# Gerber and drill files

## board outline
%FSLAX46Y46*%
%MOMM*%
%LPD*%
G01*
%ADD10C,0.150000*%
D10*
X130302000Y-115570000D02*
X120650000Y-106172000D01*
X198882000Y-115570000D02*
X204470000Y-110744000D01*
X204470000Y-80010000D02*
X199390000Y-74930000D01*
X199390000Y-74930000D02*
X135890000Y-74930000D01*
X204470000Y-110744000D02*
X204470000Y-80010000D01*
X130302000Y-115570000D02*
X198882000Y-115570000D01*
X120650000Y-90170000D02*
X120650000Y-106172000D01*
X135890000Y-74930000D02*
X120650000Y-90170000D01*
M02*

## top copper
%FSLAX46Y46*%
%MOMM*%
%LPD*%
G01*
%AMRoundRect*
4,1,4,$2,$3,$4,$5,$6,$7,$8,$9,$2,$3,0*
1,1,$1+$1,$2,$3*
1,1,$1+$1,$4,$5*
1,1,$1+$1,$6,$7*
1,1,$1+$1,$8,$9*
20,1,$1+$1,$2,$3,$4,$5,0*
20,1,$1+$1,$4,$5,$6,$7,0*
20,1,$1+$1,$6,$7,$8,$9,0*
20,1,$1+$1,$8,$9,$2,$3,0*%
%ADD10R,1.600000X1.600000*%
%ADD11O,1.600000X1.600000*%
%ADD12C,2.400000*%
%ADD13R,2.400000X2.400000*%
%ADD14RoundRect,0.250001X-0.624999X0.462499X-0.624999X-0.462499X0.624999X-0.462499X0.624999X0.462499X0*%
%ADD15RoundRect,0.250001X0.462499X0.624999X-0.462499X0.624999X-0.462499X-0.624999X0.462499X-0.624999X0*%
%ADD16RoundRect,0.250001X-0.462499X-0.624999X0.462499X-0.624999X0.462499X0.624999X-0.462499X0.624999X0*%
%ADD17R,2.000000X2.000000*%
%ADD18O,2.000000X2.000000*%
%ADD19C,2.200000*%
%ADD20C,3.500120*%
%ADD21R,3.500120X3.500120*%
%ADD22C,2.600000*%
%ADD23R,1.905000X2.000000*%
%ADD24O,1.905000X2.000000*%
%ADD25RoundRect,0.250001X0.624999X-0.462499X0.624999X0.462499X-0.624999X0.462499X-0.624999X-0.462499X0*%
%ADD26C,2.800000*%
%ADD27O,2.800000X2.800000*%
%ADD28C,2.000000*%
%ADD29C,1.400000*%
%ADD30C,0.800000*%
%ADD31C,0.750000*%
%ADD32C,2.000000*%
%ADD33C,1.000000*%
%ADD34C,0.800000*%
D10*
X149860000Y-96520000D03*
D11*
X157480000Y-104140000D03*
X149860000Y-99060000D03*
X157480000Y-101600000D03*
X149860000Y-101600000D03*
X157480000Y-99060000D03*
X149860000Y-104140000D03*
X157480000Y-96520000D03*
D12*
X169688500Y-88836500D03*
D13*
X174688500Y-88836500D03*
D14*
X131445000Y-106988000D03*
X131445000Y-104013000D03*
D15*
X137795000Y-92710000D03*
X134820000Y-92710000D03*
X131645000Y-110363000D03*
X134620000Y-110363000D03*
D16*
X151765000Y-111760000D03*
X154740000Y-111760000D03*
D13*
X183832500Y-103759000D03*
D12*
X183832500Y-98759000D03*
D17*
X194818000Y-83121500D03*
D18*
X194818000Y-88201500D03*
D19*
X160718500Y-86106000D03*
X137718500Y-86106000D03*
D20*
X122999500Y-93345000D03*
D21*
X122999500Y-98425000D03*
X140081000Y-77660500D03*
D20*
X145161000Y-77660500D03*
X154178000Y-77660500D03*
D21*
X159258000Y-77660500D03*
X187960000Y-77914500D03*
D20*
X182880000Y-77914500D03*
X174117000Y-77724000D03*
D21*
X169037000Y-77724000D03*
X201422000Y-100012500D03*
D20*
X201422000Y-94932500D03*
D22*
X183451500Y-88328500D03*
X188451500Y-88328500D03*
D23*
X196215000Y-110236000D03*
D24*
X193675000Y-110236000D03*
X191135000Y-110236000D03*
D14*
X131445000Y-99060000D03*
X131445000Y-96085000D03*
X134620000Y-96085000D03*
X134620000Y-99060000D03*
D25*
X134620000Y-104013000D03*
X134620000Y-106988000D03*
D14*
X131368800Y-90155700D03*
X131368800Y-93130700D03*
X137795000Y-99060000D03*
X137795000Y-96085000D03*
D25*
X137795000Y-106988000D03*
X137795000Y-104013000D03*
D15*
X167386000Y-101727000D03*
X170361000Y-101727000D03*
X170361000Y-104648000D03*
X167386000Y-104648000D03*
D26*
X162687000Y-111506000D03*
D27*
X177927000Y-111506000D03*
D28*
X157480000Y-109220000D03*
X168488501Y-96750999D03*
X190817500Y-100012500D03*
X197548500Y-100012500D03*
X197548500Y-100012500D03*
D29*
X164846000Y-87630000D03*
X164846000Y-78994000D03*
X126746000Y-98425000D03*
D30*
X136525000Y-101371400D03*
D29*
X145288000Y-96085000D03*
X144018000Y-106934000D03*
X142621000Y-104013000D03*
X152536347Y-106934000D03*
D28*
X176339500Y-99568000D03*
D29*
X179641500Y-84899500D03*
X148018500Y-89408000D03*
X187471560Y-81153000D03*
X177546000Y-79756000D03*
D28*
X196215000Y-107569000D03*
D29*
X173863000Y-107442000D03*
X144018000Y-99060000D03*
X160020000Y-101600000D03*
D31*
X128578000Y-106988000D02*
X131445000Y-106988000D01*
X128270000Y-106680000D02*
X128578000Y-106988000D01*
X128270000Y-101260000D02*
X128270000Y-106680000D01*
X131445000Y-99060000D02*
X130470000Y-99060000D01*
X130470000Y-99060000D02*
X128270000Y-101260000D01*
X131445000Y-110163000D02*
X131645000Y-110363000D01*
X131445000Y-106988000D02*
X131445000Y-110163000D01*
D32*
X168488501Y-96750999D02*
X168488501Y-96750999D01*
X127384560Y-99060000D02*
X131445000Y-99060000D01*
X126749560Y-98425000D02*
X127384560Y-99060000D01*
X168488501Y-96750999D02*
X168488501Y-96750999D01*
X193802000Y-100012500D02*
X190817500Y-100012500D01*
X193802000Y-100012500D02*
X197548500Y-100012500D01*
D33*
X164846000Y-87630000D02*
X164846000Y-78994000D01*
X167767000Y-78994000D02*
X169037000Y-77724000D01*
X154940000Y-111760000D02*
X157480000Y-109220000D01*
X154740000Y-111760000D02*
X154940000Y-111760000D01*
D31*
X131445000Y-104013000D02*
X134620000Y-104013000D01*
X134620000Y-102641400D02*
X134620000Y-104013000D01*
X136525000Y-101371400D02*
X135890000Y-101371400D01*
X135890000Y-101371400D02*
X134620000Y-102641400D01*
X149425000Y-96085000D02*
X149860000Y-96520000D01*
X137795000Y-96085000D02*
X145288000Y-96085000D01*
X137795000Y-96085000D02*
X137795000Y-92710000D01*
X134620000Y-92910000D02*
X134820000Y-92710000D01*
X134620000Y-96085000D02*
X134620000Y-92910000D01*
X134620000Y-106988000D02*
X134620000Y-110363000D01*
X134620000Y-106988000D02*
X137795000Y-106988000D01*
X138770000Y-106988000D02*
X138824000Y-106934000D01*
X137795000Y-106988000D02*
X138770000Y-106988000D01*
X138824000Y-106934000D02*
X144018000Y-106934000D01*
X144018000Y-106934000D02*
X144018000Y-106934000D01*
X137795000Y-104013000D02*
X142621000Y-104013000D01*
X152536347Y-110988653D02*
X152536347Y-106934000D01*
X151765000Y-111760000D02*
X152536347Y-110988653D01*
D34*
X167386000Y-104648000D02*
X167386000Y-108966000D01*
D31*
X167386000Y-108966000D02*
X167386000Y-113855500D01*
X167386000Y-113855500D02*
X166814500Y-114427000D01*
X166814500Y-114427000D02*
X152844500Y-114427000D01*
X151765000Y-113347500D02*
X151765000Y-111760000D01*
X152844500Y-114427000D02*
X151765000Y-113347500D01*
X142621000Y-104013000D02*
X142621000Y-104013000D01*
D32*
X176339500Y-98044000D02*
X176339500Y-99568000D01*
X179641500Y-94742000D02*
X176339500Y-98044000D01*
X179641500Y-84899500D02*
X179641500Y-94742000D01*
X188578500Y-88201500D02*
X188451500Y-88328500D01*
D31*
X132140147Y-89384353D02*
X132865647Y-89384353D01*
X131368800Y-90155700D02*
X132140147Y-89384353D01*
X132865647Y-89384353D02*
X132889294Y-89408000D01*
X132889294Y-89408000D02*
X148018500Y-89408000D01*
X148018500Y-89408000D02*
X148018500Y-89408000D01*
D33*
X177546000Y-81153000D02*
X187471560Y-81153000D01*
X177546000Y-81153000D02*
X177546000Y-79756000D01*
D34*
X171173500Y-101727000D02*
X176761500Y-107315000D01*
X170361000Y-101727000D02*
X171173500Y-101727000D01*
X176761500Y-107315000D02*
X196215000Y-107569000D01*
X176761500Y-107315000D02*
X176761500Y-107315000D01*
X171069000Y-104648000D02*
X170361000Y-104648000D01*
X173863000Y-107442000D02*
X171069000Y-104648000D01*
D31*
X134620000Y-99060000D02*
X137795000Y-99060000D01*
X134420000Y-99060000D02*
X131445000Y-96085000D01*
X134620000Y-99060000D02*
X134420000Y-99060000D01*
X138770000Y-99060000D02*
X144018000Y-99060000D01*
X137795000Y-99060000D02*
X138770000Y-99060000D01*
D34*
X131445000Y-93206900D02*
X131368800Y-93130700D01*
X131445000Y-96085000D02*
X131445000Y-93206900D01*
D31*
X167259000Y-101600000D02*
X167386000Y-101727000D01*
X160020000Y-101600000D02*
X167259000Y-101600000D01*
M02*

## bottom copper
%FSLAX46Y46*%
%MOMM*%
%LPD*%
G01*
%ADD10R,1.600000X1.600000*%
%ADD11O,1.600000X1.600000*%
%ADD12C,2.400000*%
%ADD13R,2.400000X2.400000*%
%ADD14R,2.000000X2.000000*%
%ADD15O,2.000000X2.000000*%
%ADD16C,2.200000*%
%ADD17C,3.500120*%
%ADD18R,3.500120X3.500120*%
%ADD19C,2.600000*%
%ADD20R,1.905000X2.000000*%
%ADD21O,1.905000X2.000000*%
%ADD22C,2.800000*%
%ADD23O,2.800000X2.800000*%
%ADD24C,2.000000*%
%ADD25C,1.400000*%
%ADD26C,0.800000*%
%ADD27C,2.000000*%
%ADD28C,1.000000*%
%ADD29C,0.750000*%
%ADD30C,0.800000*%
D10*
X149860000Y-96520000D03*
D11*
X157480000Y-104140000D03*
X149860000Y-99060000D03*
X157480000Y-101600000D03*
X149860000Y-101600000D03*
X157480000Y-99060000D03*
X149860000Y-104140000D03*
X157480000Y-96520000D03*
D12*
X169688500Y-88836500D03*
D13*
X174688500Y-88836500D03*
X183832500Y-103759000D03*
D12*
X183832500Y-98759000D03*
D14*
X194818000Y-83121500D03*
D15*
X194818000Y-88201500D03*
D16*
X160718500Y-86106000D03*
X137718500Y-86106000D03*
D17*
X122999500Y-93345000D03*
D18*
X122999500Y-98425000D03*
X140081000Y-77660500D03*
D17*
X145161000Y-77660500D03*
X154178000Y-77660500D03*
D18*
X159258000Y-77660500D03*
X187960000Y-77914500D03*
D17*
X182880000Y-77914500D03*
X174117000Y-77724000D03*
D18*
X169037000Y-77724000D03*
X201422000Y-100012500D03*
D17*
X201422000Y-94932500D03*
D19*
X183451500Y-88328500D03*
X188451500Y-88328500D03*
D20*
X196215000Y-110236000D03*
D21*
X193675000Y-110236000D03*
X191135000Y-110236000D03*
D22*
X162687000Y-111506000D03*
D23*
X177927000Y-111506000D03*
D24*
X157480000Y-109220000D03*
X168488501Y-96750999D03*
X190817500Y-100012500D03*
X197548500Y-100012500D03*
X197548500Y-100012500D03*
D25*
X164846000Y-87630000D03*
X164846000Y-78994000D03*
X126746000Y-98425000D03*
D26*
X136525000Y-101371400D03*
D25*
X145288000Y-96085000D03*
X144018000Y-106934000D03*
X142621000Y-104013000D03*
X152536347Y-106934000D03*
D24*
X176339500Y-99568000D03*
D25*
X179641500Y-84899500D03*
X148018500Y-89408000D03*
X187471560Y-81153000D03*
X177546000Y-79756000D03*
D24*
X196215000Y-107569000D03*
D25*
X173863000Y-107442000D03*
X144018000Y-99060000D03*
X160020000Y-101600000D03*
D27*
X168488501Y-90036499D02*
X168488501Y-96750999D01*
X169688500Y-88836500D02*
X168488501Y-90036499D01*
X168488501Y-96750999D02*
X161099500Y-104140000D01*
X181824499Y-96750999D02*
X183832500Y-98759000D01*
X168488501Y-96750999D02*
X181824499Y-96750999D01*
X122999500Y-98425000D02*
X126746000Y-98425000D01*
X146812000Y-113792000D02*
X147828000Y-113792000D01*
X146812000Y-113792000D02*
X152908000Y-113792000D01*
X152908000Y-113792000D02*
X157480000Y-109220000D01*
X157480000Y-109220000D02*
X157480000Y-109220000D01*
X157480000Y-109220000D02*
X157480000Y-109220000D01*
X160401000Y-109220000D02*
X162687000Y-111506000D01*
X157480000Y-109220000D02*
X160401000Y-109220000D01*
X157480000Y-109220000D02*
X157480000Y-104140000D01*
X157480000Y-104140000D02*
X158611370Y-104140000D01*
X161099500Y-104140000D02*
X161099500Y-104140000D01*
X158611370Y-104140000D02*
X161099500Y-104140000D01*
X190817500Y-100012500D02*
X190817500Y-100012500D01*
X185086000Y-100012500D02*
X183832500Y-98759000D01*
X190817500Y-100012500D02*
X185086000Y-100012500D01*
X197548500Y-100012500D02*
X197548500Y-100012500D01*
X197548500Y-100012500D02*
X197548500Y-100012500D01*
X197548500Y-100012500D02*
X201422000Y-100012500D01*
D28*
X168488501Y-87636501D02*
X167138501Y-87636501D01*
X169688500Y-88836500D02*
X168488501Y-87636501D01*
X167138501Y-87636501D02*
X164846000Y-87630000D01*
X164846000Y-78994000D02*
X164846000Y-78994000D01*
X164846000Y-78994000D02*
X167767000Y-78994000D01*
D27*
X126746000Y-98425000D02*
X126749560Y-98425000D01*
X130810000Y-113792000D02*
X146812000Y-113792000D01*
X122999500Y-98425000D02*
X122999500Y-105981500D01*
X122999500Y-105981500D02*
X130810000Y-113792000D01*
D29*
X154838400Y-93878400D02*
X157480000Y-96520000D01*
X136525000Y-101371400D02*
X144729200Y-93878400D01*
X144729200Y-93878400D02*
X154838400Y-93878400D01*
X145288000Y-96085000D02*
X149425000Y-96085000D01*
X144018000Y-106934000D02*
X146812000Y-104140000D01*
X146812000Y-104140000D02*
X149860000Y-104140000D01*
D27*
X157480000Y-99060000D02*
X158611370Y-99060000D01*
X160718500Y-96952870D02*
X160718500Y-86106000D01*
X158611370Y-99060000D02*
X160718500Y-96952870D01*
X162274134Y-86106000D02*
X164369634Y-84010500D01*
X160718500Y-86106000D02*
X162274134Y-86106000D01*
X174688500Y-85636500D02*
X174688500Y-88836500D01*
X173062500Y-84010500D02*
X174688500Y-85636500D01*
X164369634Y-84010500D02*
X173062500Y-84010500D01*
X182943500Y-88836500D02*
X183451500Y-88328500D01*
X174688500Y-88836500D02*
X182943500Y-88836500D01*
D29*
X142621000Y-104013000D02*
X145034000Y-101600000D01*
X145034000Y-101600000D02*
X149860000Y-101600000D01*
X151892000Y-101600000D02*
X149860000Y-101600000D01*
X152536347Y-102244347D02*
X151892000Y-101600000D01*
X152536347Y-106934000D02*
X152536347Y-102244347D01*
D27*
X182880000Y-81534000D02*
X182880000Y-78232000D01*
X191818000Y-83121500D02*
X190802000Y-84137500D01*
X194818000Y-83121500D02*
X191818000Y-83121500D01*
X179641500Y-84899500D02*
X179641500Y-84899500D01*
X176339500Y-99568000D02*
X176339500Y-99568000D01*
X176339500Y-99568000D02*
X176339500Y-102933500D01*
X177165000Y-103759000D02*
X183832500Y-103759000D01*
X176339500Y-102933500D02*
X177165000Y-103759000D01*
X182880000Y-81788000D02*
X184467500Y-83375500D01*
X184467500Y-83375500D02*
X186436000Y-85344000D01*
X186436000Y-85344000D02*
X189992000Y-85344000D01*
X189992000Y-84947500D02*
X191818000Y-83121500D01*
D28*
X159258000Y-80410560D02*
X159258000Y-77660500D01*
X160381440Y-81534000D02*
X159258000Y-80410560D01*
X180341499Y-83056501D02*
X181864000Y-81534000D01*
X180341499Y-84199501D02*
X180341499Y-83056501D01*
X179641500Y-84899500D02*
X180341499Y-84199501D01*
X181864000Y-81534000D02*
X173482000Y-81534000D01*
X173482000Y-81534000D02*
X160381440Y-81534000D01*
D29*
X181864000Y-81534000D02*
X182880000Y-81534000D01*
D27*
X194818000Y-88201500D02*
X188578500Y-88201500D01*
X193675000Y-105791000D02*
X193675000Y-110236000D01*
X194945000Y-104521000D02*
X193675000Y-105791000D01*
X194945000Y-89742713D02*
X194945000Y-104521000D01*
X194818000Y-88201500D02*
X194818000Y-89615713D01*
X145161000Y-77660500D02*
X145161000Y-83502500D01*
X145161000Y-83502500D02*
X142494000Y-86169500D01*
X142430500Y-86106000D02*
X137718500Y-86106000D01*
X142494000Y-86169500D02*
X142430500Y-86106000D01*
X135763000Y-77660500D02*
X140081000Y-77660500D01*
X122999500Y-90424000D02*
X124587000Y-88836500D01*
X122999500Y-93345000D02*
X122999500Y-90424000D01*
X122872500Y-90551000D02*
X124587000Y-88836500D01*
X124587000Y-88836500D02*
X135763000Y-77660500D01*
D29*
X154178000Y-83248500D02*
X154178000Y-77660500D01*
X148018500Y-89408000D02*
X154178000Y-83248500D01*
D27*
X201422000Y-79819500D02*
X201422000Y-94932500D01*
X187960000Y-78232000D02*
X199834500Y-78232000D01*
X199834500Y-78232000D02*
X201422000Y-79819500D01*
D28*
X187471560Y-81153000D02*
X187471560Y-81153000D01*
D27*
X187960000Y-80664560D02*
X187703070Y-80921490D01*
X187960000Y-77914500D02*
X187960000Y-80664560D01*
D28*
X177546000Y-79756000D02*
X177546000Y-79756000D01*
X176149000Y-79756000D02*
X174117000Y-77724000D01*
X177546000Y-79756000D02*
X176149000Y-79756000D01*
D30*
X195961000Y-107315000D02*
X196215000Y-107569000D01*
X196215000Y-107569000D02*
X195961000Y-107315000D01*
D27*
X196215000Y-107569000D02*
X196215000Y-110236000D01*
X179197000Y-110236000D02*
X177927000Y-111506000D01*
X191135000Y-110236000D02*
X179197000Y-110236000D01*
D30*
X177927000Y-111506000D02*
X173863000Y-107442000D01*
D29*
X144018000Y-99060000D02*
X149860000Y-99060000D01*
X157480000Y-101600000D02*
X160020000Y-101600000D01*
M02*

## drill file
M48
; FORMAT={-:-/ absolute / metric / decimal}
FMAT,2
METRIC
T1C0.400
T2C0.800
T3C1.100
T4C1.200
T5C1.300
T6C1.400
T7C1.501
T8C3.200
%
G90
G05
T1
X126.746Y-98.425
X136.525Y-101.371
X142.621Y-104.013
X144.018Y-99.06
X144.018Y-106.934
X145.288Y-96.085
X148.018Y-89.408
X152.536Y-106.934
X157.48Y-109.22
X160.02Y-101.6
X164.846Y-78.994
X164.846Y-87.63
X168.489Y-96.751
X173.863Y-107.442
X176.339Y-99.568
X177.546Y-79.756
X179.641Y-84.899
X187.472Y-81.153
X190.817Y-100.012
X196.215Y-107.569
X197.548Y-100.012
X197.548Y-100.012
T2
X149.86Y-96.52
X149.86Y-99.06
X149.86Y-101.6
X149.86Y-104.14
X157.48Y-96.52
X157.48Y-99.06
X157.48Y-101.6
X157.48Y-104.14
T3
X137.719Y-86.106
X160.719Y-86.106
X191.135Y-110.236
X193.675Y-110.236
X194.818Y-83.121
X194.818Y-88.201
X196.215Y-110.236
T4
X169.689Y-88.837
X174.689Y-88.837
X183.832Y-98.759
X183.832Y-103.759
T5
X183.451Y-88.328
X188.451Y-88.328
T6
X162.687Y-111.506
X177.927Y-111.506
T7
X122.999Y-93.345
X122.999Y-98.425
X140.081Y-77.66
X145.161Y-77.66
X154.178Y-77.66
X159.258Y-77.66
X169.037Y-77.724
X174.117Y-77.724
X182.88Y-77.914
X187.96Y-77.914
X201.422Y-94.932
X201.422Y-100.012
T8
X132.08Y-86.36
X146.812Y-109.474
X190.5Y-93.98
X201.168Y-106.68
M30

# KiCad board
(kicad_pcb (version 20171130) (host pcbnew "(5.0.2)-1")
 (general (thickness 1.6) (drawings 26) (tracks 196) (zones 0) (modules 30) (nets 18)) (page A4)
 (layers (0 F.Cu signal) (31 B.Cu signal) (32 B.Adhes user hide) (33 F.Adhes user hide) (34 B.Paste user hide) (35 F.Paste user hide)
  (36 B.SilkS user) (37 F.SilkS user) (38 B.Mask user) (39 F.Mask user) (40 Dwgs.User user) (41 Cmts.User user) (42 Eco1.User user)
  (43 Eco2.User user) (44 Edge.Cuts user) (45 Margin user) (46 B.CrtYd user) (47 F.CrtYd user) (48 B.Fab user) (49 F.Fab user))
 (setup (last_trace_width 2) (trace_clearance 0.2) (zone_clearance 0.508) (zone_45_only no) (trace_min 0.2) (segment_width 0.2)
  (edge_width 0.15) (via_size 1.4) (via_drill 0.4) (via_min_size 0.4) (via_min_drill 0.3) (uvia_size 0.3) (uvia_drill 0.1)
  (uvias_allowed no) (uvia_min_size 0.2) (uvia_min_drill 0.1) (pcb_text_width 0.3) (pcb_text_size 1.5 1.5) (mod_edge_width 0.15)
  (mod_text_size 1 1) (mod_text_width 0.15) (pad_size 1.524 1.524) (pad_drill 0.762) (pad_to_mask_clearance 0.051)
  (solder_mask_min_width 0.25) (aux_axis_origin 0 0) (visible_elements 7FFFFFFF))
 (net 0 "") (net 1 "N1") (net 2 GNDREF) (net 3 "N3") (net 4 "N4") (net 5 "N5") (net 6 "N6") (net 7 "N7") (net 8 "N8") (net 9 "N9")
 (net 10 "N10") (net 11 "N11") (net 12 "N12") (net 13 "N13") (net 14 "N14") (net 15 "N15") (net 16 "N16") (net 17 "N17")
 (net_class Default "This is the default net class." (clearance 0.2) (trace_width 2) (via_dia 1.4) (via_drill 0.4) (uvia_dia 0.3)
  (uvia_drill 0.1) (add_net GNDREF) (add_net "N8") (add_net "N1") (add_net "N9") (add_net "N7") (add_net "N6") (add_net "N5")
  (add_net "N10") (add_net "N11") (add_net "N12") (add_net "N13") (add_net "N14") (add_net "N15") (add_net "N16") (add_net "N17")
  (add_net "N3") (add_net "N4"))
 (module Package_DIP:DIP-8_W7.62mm (layer F.Cu) (at 149.86 96.52)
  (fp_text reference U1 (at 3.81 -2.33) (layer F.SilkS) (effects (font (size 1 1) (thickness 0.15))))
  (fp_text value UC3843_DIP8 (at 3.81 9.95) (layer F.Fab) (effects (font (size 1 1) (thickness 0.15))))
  (pad 1 thru_hole rect (at 0 0) (size 1.6 1.6) (drill 0.8) (layers *.Cu *.Mask) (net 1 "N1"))
  (pad 5 thru_hole oval (at 7.62 7.62) (size 1.6 1.6) (drill 0.8) (layers *.Cu *.Mask) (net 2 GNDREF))
  (pad 2 thru_hole oval (at 0 2.54) (size 1.6 1.6) (drill 0.8) (layers *.Cu *.Mask) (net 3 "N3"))
  (pad 6 thru_hole oval (at 7.62 5.08) (size 1.6 1.6) (drill 0.8) (layers *.Cu *.Mask) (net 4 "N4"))
  (pad 3 thru_hole oval (at 0 5.08) (size 1.6 1.6) (drill 0.8) (layers *.Cu *.Mask) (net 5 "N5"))
  (pad 7 thru_hole oval (at 7.62 2.54) (size 1.6 1.6) (drill 0.8) (layers *.Cu *.Mask) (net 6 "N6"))
  (pad 4 thru_hole oval (at 0 7.62) (size 1.6 1.6) (drill 0.8) (layers *.Cu *.Mask) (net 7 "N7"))
  (pad 8 thru_hole oval (at 7.62 0) (size 1.6 1.6) (drill 0.8) (layers *.Cu *.Mask) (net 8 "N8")))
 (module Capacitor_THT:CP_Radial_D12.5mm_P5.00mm (layer F.Cu) (at 174.6885 88.8365 180)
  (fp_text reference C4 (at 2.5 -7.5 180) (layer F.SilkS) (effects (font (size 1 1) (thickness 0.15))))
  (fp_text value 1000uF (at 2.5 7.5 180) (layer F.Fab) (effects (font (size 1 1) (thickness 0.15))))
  (pad 2 thru_hole circle (at 5 0 180) (size 2.4 2.4) (drill 1.2) (layers *.Cu *.Mask) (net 2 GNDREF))
  (pad 1 thru_hole rect (at 0 0 180) (size 2.4 2.4) (drill 1.2) (layers *.Cu *.Mask) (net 6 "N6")))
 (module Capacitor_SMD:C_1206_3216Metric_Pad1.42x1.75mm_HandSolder (layer F.Cu) (at 131.445 105.5005 270)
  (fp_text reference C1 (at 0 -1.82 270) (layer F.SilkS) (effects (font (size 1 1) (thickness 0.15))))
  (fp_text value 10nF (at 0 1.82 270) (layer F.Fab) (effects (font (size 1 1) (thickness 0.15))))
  (pad 2 smd roundrect (at 1.4875 0 270) (size 1.425 1.75) (layers F.Cu F.Paste F.Mask) (roundrect_rratio 0.175439) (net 2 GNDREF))
  (pad 1 smd roundrect (at -1.4875 0 270) (size 1.425 1.75) (layers F.Cu F.Paste F.Mask) (roundrect_rratio 0.175439) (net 8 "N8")))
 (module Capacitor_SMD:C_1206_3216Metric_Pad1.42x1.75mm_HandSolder (layer F.Cu) (at 136.3075 92.71 180)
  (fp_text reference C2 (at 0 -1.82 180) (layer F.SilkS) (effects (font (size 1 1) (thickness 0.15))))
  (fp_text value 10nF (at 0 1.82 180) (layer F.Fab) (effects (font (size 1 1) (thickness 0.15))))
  (pad 1 smd roundrect (at -1.4875 0 180) (size 1.425 1.75) (layers F.Cu F.Paste F.Mask) (roundrect_rratio 0.175439) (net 1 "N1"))
  (pad 2 smd roundrect (at 1.4875 0 180) (size 1.425 1.75) (layers F.Cu F.Paste F.Mask) (roundrect_rratio 0.175439) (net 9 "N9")))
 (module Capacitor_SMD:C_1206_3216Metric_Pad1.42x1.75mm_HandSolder (layer F.Cu) (at 133.1325 110.363 180)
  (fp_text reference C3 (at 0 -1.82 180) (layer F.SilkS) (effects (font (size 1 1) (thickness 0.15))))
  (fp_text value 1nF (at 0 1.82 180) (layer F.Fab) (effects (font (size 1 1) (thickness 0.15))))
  (pad 2 smd roundrect (at 1.4875 0 180) (size 1.425 1.75) (layers F.Cu F.Paste F.Mask) (roundrect_rratio 0.175439) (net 2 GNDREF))
  (pad 1 smd roundrect (at -1.4875 0 180) (size 1.425 1.75) (layers F.Cu F.Paste F.Mask) (roundrect_rratio 0.175439) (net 7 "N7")))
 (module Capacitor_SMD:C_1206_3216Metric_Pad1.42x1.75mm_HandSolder (layer F.Cu) (at 153.2525 111.76)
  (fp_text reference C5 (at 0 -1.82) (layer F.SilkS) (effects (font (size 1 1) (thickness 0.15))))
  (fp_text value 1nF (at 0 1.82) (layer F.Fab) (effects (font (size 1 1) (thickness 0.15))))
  (pad 1 smd roundrect (at -1.4875 0) (size 1.425 1.75) (layers F.Cu F.Paste F.Mask) (roundrect_rratio 0.175439) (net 5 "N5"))
  (pad 2 smd roundrect (at 1.4875 0) (size 1.425 1.75) (layers F.Cu F.Paste F.Mask) (roundrect_rratio 0.175439) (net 2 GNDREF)))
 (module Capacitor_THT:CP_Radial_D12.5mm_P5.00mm (layer F.Cu) (at 183.8325 103.759 90)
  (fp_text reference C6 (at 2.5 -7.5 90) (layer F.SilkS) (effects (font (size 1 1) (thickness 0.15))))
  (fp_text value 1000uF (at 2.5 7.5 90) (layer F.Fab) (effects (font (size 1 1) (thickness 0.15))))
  (pad 1 thru_hole rect (at 0 0 90) (size 2.4 2.4) (drill 1.2) (layers *.Cu *.Mask) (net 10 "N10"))
  (pad 2 thru_hole circle (at 5 0 90) (size 2.4 2.4) (drill 1.2) (layers *.Cu *.Mask) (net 2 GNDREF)))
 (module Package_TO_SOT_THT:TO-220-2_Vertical (layer F.Cu) (at 194.818 83.1215 270)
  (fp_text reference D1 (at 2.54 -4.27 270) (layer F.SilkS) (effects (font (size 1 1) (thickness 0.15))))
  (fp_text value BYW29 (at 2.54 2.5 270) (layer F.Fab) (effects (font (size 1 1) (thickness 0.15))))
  (pad 1 thru_hole rect (at 0 0 270) (size 2 2) (drill 1.1) (layers *.Cu *.Mask) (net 10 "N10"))
  (pad 2 thru_hole oval (at 5.08 0 270) (size 2 2) (drill 1.1) (layers *.Cu *.Mask) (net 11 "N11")))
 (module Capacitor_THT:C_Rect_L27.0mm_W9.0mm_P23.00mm (layer F.Cu) (at 160.7185 86.106 180)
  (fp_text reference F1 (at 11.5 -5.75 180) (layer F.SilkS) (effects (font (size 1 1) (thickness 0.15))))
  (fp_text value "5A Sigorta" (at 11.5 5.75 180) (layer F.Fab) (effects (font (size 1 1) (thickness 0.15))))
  (pad 1 thru_hole circle (at 0 0 180) (size 2.2 2.2) (drill 1.1) (layers *.Cu *.Mask) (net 6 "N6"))
  (pad 2 thru_hole circle (at 23 0 180) (size 2.2 2.2) (drill 1.1) (layers *.Cu *.Mask) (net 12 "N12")))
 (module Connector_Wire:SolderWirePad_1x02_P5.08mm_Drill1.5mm (layer F.Cu) (at 122.9995 98.425 90)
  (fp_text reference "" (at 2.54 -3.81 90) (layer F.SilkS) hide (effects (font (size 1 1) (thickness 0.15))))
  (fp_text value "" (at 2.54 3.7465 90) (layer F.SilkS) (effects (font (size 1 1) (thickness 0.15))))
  (pad 2 thru_hole circle (at 5.08 0 90) (size 3.50012 3.50012) (drill 1.50114) (layers *.Cu *.Mask) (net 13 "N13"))
  (pad 1 thru_hole rect (at 0 0 90) (size 3.50012 3.50012) (drill 1.50114) (layers *.Cu *.Mask) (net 2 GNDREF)))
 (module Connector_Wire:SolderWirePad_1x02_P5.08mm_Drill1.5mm (layer F.Cu) (at 140.081 77.6605)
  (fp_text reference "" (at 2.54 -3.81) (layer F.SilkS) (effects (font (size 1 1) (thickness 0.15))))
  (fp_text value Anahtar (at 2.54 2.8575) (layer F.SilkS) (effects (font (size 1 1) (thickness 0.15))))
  (pad 1 thru_hole rect (at 0 0) (size 3.50012 3.50012) (drill 1.50114) (layers *.Cu *.Mask) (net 13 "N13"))
  (pad 2 thru_hole circle (at 5.08 0) (size 3.50012 3.50012) (drill 1.50114) (layers *.Cu *.Mask) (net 12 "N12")))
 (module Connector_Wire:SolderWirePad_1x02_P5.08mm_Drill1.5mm (layer F.Cu) (at 159.258 77.6605 180)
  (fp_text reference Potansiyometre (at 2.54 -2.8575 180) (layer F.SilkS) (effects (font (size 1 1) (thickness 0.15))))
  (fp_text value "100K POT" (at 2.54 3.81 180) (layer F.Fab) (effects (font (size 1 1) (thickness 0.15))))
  (pad 2 thru_hole circle (at 5.08 0 180) (size 3.50012 3.50012) (drill 1.50114) (layers *.Cu *.Mask) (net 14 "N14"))
  (pad 1 thru_hole rect (at 0 0 180) (size 3.50012 3.50012) (drill 1.50114) (layers *.Cu *.Mask) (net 10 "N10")))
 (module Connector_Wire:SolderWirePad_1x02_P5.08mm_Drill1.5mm (layer F.Cu) (at 187.96 77.9145 180)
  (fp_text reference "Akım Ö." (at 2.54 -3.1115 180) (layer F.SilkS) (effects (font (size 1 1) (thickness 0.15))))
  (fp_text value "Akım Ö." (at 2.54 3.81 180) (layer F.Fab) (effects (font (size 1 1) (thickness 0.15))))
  (pad 1 thru_hole rect (at 0 0 180) (size 3.50012 3.50012) (drill 1.50114) (layers *.Cu *.Mask) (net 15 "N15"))
  (pad 2 thru_hole circle (at 5.08 0 180) (size 3.50012 3.50012) (drill 1.50114) (layers *.Cu *.Mask) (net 10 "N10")))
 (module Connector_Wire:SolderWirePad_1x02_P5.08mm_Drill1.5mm (layer F.Cu) (at 169.037 77.724)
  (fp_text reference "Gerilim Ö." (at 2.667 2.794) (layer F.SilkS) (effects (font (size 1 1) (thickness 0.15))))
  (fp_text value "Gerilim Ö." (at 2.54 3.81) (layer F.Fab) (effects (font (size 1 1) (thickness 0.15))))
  (pad 2 thru_hole circle (at 5.08 0) (size 3.50012 3.50012) (drill 1.50114) (layers *.Cu *.Mask) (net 15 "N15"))
  (pad 1 thru_hole rect (at 0 0) (size 3.50012 3.50012) (drill 1.50114) (layers *.Cu *.Mask) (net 2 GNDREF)))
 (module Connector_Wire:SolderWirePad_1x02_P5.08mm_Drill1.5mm (layer F.Cu) (at 201.422 100.0125 90)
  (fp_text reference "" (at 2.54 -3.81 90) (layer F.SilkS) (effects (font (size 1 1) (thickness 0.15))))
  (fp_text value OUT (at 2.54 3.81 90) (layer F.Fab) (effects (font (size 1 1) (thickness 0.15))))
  (pad 1 thru_hole rect (at 0 0 90) (size 3.50012 3.50012) (drill 1.50114) (layers *.Cu *.Mask) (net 2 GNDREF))
  (pad 2 thru_hole circle (at 5.08 0 90) (size 3.50012 3.50012) (drill 1.50114) (layers *.Cu *.Mask) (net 15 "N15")))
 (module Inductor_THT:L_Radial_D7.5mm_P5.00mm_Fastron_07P (layer F.Cu) (at 183.4515 88.3285)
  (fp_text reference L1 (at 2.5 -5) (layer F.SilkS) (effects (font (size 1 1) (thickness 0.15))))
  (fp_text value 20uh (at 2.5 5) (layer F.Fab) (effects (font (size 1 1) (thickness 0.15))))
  (pad 1 thru_hole circle (at 0 0) (size 2.6 2.6) (drill 1.3) (layers *.Cu *.Mask) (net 6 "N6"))
  (pad 2 thru_hole circle (at 5 0) (size 2.6 2.6) (drill 1.3) (layers *.Cu *.Mask) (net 11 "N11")))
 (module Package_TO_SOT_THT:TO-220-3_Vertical (layer F.Cu) (at 196.215 110.236 180)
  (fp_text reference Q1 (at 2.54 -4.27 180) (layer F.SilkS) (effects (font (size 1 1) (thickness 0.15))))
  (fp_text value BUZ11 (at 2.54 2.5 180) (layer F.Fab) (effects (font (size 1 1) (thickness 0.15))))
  (pad 1 thru_hole rect (at 0 0 180) (size 1.905 2) (drill 1.1) (layers *.Cu *.Mask) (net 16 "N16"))
  (pad 2 thru_hole oval (at 2.54 0 180) (size 1.905 2) (drill 1.1) (layers *.Cu *.Mask) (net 11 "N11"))
  (pad 3 thru_hole oval (at 5.08 0 180) (size 1.905 2) (drill 1.1) (layers *.Cu *.Mask) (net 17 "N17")))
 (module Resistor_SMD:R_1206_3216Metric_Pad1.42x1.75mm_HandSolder (layer F.Cu) (at 131.445 97.5725 270)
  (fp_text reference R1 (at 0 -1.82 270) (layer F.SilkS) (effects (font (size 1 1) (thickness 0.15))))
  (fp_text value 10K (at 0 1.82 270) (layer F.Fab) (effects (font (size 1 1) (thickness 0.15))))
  (pad 2 smd roundrect (at 1.4875 0 270) (size 1.425 1.75) (layers F.Cu F.Paste F.Mask) (roundrect_rratio 0.175439) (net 2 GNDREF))
  (pad 1 smd roundrect (at -1.4875 0 270) (size 1.425 1.75) (layers F.Cu F.Paste F.Mask) (roundrect_rratio 0.175439) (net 3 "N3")))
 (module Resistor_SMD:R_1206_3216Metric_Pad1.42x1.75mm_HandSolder (layer F.Cu) (at 134.62 97.5725 270)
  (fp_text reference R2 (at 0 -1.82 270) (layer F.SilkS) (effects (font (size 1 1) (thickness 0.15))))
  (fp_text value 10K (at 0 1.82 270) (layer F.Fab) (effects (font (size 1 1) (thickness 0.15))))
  (pad 1 smd roundrect (at -1.4875 0 270) (size 1.425 1.75) (layers F.Cu F.Paste F.Mask) (roundrect_rratio 0.175439) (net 9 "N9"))
  (pad 2 smd roundrect (at 1.4875 0 270) (size 1.425 1.75) (layers F.Cu F.Paste F.Mask) (roundrect_rratio 0.175439) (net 3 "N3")))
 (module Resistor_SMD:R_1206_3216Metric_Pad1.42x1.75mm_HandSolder (layer F.Cu) (at 134.62 105.5005 90)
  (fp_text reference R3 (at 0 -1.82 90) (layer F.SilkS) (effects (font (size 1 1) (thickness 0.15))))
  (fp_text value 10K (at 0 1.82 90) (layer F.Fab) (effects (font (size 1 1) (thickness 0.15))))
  (pad 2 smd roundrect (at 1.4875 0 90) (size 1.425 1.75) (layers F.Cu F.Paste F.Mask) (roundrect_rratio 0.175439) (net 8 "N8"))
  (pad 1 smd roundrect (at -1.4875 0 90) (size 1.425 1.75) (layers F.Cu F.Paste F.Mask) (roundrect_rratio 0.175439) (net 7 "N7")))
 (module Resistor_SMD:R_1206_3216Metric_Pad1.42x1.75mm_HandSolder (layer F.Cu) (at 131.3688 91.6432 270)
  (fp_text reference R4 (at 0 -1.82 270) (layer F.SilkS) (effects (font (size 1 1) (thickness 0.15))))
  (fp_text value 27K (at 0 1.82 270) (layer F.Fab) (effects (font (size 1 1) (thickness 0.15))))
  (pad 1 smd roundrect (at -1.4875 0 270) (size 1.425 1.75) (layers F.Cu F.Paste F.Mask) (roundrect_rratio 0.175439) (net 14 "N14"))
  (pad 2 smd roundrect (at 1.4875 0 270) (size 1.425 1.75) (layers F.Cu F.Paste F.Mask) (roundrect_rratio 0.175439) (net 3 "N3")))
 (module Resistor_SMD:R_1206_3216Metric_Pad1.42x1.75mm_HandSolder (layer F.Cu) (at 137.795 97.5725 270)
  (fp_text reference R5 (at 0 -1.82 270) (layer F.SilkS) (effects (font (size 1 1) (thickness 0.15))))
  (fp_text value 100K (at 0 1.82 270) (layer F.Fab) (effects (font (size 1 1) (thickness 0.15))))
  (pad 2 smd roundrect (at 1.4875 0 270) (size 1.425 1.75) (layers F.Cu F.Paste F.Mask) (roundrect_rratio 0.175439) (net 3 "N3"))
  (pad 1 smd roundrect (at -1.4875 0 270) (size 1.425 1.75) (layers F.Cu F.Paste F.Mask) (roundrect_rratio 0.175439) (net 1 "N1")))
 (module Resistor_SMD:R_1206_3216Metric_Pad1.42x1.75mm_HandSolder (layer F.Cu) (at 137.795 105.5005 90)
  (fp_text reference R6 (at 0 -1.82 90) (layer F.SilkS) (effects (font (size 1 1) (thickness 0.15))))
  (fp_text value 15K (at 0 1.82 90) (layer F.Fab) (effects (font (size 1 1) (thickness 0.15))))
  (pad 1 smd roundrect (at -1.4875 0 90) (size 1.425 1.75) (layers F.Cu F.Paste F.Mask) (roundrect_rratio 0.175439) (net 7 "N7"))
  (pad 2 smd roundrect (at 1.4875 0 90) (size 1.425 1.75) (layers F.Cu F.Paste F.Mask) (roundrect_rratio 0.175439) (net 5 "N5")))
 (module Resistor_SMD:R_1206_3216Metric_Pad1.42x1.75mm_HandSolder (layer F.Cu) (at 168.8735 101.727 180)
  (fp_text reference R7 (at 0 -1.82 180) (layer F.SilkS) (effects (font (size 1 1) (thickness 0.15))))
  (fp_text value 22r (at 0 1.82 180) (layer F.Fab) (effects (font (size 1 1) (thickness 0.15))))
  (pad 2 smd roundrect (at 1.4875 0 180) (size 1.425 1.75) (layers F.Cu F.Paste F.Mask) (roundrect_rratio 0.175439) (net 4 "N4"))
  (pad 1 smd roundrect (at -1.4875 0 180) (size 1.425 1.75) (layers F.Cu F.Paste F.Mask) (roundrect_rratio 0.175439) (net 16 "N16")))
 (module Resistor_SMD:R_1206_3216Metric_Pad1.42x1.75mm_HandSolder (layer F.Cu) (at 168.8735 104.648 180)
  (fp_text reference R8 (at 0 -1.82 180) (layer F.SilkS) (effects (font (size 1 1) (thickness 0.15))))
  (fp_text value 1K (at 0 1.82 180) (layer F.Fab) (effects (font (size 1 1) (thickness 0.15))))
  (pad 1 smd roundrect (at -1.4875 0 180) (size 1.425 1.75) (layers F.Cu F.Paste F.Mask) (roundrect_rratio 0.175439) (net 17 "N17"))
  (pad 2 smd roundrect (at 1.4875 0 180) (size 1.425 1.75) (layers F.Cu F.Paste F.Mask) (roundrect_rratio 0.175439) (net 5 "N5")))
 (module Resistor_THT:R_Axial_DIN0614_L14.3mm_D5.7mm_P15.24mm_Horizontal (layer F.Cu) (at 162.687 111.506)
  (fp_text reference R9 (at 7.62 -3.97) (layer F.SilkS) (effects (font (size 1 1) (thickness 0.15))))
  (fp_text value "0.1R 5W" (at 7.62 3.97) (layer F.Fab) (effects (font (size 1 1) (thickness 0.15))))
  (pad 1 thru_hole circle (at 0 0) (size 2.8 2.8) (drill 1.4) (layers *.Cu *.Mask) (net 2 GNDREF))
  (pad 2 thru_hole oval (at 15.24 0) (size 2.8 2.8) (drill 1.4) (layers *.Cu *.Mask) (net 17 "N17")))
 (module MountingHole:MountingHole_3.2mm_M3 (layer F.Cu) (at 132.08 86.36)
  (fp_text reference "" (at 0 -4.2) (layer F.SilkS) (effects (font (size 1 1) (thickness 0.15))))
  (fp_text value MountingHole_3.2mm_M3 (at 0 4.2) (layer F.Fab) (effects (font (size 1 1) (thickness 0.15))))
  (pad 1 np_thru_hole circle (at 0 0) (size 3.2 3.2) (drill 3.2) (layers *.Cu *.Mask)))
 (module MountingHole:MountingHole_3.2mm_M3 (layer F.Cu) (at 201.168 106.68)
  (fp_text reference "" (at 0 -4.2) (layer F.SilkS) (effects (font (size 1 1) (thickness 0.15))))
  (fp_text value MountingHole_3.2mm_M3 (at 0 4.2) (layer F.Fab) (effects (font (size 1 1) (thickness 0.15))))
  (pad 1 np_thru_hole circle (at 0 0) (size 3.2 3.2) (drill 3.2) (layers *.Cu *.Mask)))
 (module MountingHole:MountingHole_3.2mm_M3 (layer F.Cu) (at 190.5 93.98)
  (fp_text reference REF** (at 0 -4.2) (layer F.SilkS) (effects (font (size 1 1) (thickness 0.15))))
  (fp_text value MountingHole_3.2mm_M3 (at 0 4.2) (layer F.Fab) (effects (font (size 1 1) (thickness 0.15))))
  (pad 1 np_thru_hole circle (at 0 0) (size 3.2 3.2) (drill 3.2) (layers *.Cu *.Mask)))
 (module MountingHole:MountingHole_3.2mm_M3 (layer F.Cu) (at 146.812 109.474)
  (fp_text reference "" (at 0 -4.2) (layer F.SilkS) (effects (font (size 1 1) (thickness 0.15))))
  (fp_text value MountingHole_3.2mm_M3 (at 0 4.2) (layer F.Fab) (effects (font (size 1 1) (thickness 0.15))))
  (pad 1 np_thru_hole circle (at 0 0) (size 3.2 3.2) (drill 3.2) (layers *.Cu *.Mask)))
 (gr_line (start 130.302 115.57) (end 120.65 106.172) (layer Edge.Cuts) (width 0.15))
 (gr_line (start 198.882 115.57) (end 204.47 110.744) (layer Edge.Cuts) (width 0.15))
 (gr_line (start 204.47 80.01) (end 199.39 74.93) (layer Edge.Cuts) (width 0.15))
 (gr_line (start 199.39 74.93) (end 135.89 74.93) (layer Edge.Cuts) (width 0.15))
 (gr_line (start 204.47 110.744) (end 204.47 80.01) (layer Edge.Cuts) (width 0.15))
 (gr_line (start 130.302 115.57) (end 198.882 115.57) (layer Edge.Cuts) (width 0.15))
 (gr_line (start 120.65 90.17) (end 120.65 106.172) (layer Edge.Cuts) (width 0.15))
 (gr_line (start 135.89 74.93) (end 120.65 90.17) (layer Edge.Cuts) (width 0.15))
 (segment (start 128.578 106.988) (end 131.445 106.988) (width 0.75) (layer F.Cu) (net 2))
 (segment (start 128.27 106.68) (end 128.578 106.988) (width 0.75) (layer F.Cu) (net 2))
 (segment (start 128.27 101.26) (end 128.27 106.68) (width 0.75) (layer F.Cu) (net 2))
 (segment (start 131.445 99.06) (end 130.47 99.06) (width 0.75) (layer F.Cu) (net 2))
 (segment (start 130.47 99.06) (end 128.27 101.26) (width 0.75) (layer F.Cu) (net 2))
 (segment (start 131.445 110.163) (end 131.645 110.363) (width 0.75) (layer F.Cu) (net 2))
 (segment (start 131.445 106.988) (end 131.445 110.163) (width 0.75) (layer F.Cu) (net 2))
 (segment (start 168.488501 90.036499) (end 168.488501 96.750999) (width 2) (layer B.Cu) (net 2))
 (segment (start 169.6885 88.8365) (end 168.488501 90.036499) (width 2) (layer B.Cu) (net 2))
 (segment (start 168.488501 96.750999) (end 161.0995 104.14) (width 2) (layer B.Cu) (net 2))
 (segment (start 181.824499 96.750999) (end 183.8325 98.759) (width 2) (layer B.Cu) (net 2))
 (segment (start 168.488501 96.750999) (end 181.824499 96.750999) (width 2) (layer B.Cu) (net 2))
 (segment (start 168.488501 96.750999) (end 168.488501 96.750999) (width 2) (layer F.Cu) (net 2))
 (segment (start 122.9995 98.425) (end 126.746 98.425) (width 2) (layer B.Cu) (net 2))
 (segment (start 127.38456 99.06) (end 131.445 99.06) (width 2) (layer F.Cu) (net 2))
 (segment (start 126.74956 98.425) (end 127.38456 99.06) (width 2) (layer F.Cu) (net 2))
 (segment (start 146.812 113.792) (end 147.828 113.792) (width 2) (layer B.Cu) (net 2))
 (segment (start 146.812 113.792) (end 152.908 113.792) (width 2) (layer B.Cu) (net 2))
 (segment (start 152.908 113.792) (end 157.48 109.22) (width 2) (layer B.Cu) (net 2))
 (segment (start 157.48 109.22) (end 157.48 109.22) (width 2) (layer B.Cu) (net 2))
 (segment (start 157.48 109.22) (end 157.48 109.22) (width 2) (layer B.Cu) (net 2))
 (via (at 157.48 109.22) (size 2) (drill 0.4) (layers F.Cu B.Cu) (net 2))
 (segment (start 160.401 109.22) (end 162.687 111.506) (width 2) (layer B.Cu) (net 2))
 (segment (start 157.48 109.22) (end 160.401 109.22) (width 2) (layer B.Cu) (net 2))
 (segment (start 157.48 109.22) (end 157.48 104.14) (width 2) (layer B.Cu) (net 2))
 (segment (start 157.48 104.14) (end 158.61137 104.14) (width 2) (layer B.Cu) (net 2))
 (segment (start 161.0995 104.14) (end 161.0995 104.14) (width 2) (layer B.Cu) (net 2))
 (segment (start 158.61137 104.14) (end 161.0995 104.14) (width 2) (layer B.Cu) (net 2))
 (segment (start 168.488501 96.750999) (end 168.488501 96.750999) (width 2) (layer F.Cu) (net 2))
 (via (at 168.488501 96.750999) (size 2) (drill 0.4) (layers F.Cu B.Cu) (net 2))
 (segment (start 193.802 100.0125) (end 190.8175 100.0125) (width 2) (layer F.Cu) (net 2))
 (segment (start 190.8175 100.0125) (end 190.8175 100.0125) (width 2) (layer B.Cu) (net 2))
 (via (at 190.8175 100.0125) (size 2) (drill 0.4) (layers F.Cu B.Cu) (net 2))
 (segment (start 185.086 100.0125) (end 183.8325 98.759) (width 2) (layer B.Cu) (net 2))
 (segment (start 190.8175 100.0125) (end 185.086 100.0125) (width 2) (layer B.Cu) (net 2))
 (segment (start 193.802 100.0125) (end 197.5485 100.0125) (width 2) (layer F.Cu) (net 2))
 (segment (start 197.5485 100.0125) (end 197.5485 100.0125) (width 2) (layer B.Cu) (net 2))
 (via (at 197.5485 100.0125) (size 2) (drill 0.4) (layers F.Cu B.Cu) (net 2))
 (segment (start 197.5485 100.0125) (end 197.5485 100.0125) (width 2) (layer B.Cu) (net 2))
 (via (at 197.5485 100.0125) (size 2) (drill 0.4) (layers F.Cu B.Cu) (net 2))
 (segment (start 197.5485 100.0125) (end 201.422 100.0125) (width 2) (layer B.Cu) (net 2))
 (segment (start 168.488501 87.636501) (end 167.138501 87.636501) (width 1) (layer B.Cu) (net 2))
 (segment (start 169.6885 88.8365) (end 168.488501 87.636501) (width 1) (layer B.Cu) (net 2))
 (segment (start 167.138501 87.636501) (end 164.846 87.63) (width 1) (layer B.Cu) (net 2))
 (via (at 164.846 87.63) (size 1.4) (drill 0.4) (layers F.Cu B.Cu) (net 2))
 (segment (start 164.846 87.63) (end 164.846 78.994) (width 1) (layer F.Cu) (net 2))
 (segment (start 164.846 78.994) (end 164.846 78.994) (width 1) (layer B.Cu) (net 2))
 (via (at 164.846 78.994) (size 1.4) (drill 0.4) (layers F.Cu B.Cu) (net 2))
 (segment (start 167.767 78.994) (end 169.037 77.724) (width 1) (layer F.Cu) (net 2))
 (segment (start 164.846 78.994) (end 167.767 78.994) (width 1) (layer B.Cu) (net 2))
 (segment (start 154.94 111.76) (end 157.48 109.22) (width 1) (layer F.Cu) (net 2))
 (segment (start 154.74 111.76) (end 154.94 111.76) (width 1) (layer F.Cu) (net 2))
 (segment (start 126.746 98.425) (end 126.74956 98.425) (width 2) (layer B.Cu) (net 2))
 (via (at 126.746 98.425) (size 1.4) (drill 0.4) (layers F.Cu B.Cu) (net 2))
 (segment (start 130.81 113.792) (end 146.812 113.792) (width 2) (layer B.Cu) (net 2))
 (segment (start 122.9995 98.425) (end 122.9995 105.9815) (width 2) (layer B.Cu) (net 2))
 (segment (start 122.9995 105.9815) (end 130.81 113.792) (width 2) (layer B.Cu) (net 2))
 (via (at 136.525 101.3714) (size 0.8) (drill 0.4) (layers F.Cu B.Cu) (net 8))
 (segment (start 131.445 104.013) (end 134.62 104.013) (width 0.75) (layer F.Cu) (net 8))
 (segment (start 134.62 102.6414) (end 134.62 104.013) (width 0.75) (layer F.Cu) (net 8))
 (segment (start 136.525 101.3714) (end 135.89 101.3714) (width 0.75) (layer F.Cu) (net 8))
 (segment (start 135.89 101.3714) (end 134.62 102.6414) (width 0.75) (layer F.Cu) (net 8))
 (segment (start 154.8384 93.8784) (end 157.48 96.52) (width 0.75) (layer B.Cu) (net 8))
 (segment (start 136.525 101.3714) (end 144.7292 93.8784) (width 0.75) (layer B.Cu) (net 8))
 (segment (start 144.7292 93.8784) (end 154.8384 93.8784) (width 0.75) (layer B.Cu) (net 8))
 (segment (start 149.425 96.085) (end 149.86 96.52) (width 0.75) (layer F.Cu) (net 1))
 (segment (start 137.795 96.085) (end 145.288 96.085) (width 0.75) (layer F.Cu) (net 1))
 (segment (start 137.795 96.085) (end 137.795 92.71) (width 0.75) (layer F.Cu) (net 1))
 (segment (start 145.288 96.085) (end 149.425 96.085) (width 0.75) (layer B.Cu) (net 1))
 (via (at 145.288 96.085) (size 1.4) (drill 0.4) (layers F.Cu B.Cu) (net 1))
 (segment (start 134.62 92.91) (end 134.82 92.71) (width 0.75) (layer F.Cu) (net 9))
 (segment (start 134.62 96.085) (end 134.62 92.91) (width 0.75) (layer F.Cu) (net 9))
 (segment (start 134.62 106.988) (end 134.62 110.363) (width 0.75) (layer F.Cu) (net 7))
 (segment (start 134.62 106.988) (end 137.795 106.988) (width 0.75) (layer F.Cu) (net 7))
 (segment (start 138.77 106.988) (end 138.824 106.934) (width 0.75) (layer F.Cu) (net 7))
 (segment (start 137.795 106.988) (end 138.77 106.988) (width 0.75) (layer F.Cu) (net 7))
 (segment (start 138.824 106.934) (end 144.018 106.934) (width 0.75) (layer F.Cu) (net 7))
 (segment (start 144.018 106.934) (end 146.812 104.14) (width 0.75) (layer B.Cu) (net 7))
 (segment (start 146.812 104.14) (end 149.86 104.14) (width 0.75) (layer B.Cu) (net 7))
 (segment (start 144.018 106.934) (end 144.018 106.934) (width 0.75) (layer F.Cu) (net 7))
 (via (at 144.018 106.934) (size 1.4) (drill 0.4) (layers F.Cu B.Cu) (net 7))
 (segment (start 157.48 99.06) (end 158.61137 99.06) (width 2) (layer B.Cu) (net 6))
 (segment (start 160.7185 96.95287) (end 160.7185 86.106) (width 2) (layer B.Cu) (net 6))
 (segment (start 158.61137 99.06) (end 160.7185 96.95287) (width 2) (layer B.Cu) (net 6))
 (segment (start 162.274134 86.106) (end 164.369634 84.0105) (width 2) (layer B.Cu) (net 6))
 (segment (start 160.7185 86.106) (end 162.274134 86.106) (width 2) (layer B.Cu) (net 6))
 (segment (start 174.6885 85.6365) (end 174.6885 88.8365) (width 2) (layer B.Cu) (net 6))
 (segment (start 173.0625 84.0105) (end 174.6885 85.6365) (width 2) (layer B.Cu) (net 6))
 (segment (start 164.369634 84.0105) (end 173.0625 84.0105) (width 2) (layer B.Cu) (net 6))
 (segment (start 182.9435 88.8365) (end 183.4515 88.3285) (width 2) (layer B.Cu) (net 6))
 (segment (start 174.6885 88.8365) (end 182.9435 88.8365) (width 2) (layer B.Cu) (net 6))
 (segment (start 137.795 104.013) (end 142.621 104.013) (width 0.75) (layer F.Cu) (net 5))
 (segment (start 142.621 104.013) (end 145.034 101.6) (width 0.75) (layer B.Cu) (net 5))
 (segment (start 145.034 101.6) (end 149.86 101.6) (width 0.75) (layer B.Cu) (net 5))
 (segment (start 152.536347 110.988653) (end 152.536347 106.934) (width 0.75) (layer F.Cu) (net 5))
 (segment (start 151.765 111.76) (end 152.536347 110.988653) (width 0.75) (layer F.Cu) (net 5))
 (segment (start 151.892 101.6) (end 149.86 101.6) (width 0.75) (layer B.Cu) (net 5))
 (segment (start 152.536347 102.244347) (end 151.892 101.6) (width 0.75) (layer B.Cu) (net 5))
 (segment (start 167.386 104.648) (end 167.386 108.966) (width 0.8) (layer F.Cu) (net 5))
 (segment (start 167.386 108.966) (end 167.386 113.8555) (width 0.75) (layer F.Cu) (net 5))
 (segment (start 167.386 113.8555) (end 166.8145 114.427) (width 0.75) (layer F.Cu) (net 5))
 (segment (start 166.8145 114.427) (end 152.8445 114.427) (width 0.75) (layer F.Cu) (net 5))
 (segment (start 151.765 113.3475) (end 151.765 111.76) (width 0.75) (layer F.Cu) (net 5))
 (segment (start 152.8445 114.427) (end 151.765 113.3475) (width 0.75) (layer F.Cu) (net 5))
 (segment (start 142.621 104.013) (end 142.621 104.013) (width 0.75) (layer F.Cu) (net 5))
 (via (at 142.621 104.013) (size 1.4) (drill 0.4) (layers F.Cu B.Cu) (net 5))
 (segment (start 152.536347 106.934) (end 152.536347 102.244347) (width 0.75) (layer B.Cu) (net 5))
 (via (at 152.536347 106.934) (size 1.4) (drill 0.4) (layers F.Cu B.Cu) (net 5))
 (segment (start 182.88 81.534) (end 182.88 78.232) (width 2) (layer B.Cu) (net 10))
 (segment (start 176.3395 98.044) (end 176.3395 99.568) (width 2) (layer F.Cu) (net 10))
 (segment (start 179.6415 94.742) (end 176.3395 98.044) (width 2) (layer F.Cu) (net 10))
 (segment (start 191.818 83.1215) (end 190.802 84.1375) (width 2) (layer B.Cu) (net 10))
 (segment (start 194.818 83.1215) (end 191.818 83.1215) (width 2) (layer B.Cu) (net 10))
 (segment (start 179.6415 84.8995) (end 179.6415 84.8995) (width 2) (layer B.Cu) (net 10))
 (segment (start 176.3395 99.568) (end 176.3395 99.568) (width 2) (layer B.Cu) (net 10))
 (via (at 176.3395 99.568) (size 2) (drill 0.4) (layers F.Cu B.Cu) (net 10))
 (segment (start 176.3395 99.568) (end 176.3395 102.9335) (width 2) (layer B.Cu) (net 10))
 (segment (start 177.165 103.759) (end 183.8325 103.759) (width 2) (layer B.Cu) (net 10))
 (segment (start 176.3395 102.9335) (end 177.165 103.759) (width 2) (layer B.Cu) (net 10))
 (segment (start 182.88 81.788) (end 184.4675 83.3755) (width 2) (layer B.Cu) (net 10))
 (segment (start 184.4675 83.3755) (end 186.436 85.344) (width 2) (layer B.Cu) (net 10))
 (segment (start 186.436 85.344) (end 189.992 85.344) (width 2) (layer B.Cu) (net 10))
 (segment (start 189.992 84.9475) (end 191.818 83.1215) (width 2) (layer B.Cu) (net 10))
 (segment (start 159.258 80.41056) (end 159.258 77.6605) (width 1) (layer B.Cu) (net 10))
 (segment (start 160.38144 81.534) (end 159.258 80.41056) (width 1) (layer B.Cu) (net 10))
 (segment (start 179.6415 84.8995) (end 179.6415 94.742) (width 2) (layer F.Cu) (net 10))
 (via (at 179.6415 84.8995) (size 1.4) (drill 0.4) (layers F.Cu B.Cu) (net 10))
 (segment (start 180.341499 83.056501) (end 181.864 81.534) (width 1) (layer B.Cu) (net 10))
 (segment (start 180.341499 84.199501) (end 180.341499 83.056501) (width 1) (layer B.Cu) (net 10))
 (segment (start 179.6415 84.8995) (end 180.341499 84.199501) (width 1) (layer B.Cu) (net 10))
 (segment (start 181.864 81.534) (end 173.482 81.534) (width 1) (layer B.Cu) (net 10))
 (segment (start 173.482 81.534) (end 160.38144 81.534) (width 1) (layer B.Cu) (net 10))
 (segment (start 181.864 81.534) (end 182.88 81.534) (width 0.75) (layer B.Cu) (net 10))
 (segment (start 188.5785 88.2015) (end 188.4515 88.3285) (width 2) (layer F.Cu) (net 11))
 (segment (start 194.818 88.2015) (end 188.5785 88.2015) (width 2) (layer B.Cu) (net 11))
 (segment (start 193.675 105.791) (end 193.675 110.236) (width 2) (layer B.Cu) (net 11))
 (segment (start 194.945 104.521) (end 193.675 105.791) (width 2) (layer B.Cu) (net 11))
 (segment (start 194.945 89.742713) (end 194.945 104.521) (width 2) (layer B.Cu) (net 11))
 (segment (start 194.818 88.2015) (end 194.818 89.615713) (width 2) (layer B.Cu) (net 11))
 (segment (start 145.161 77.6605) (end 145.161 83.5025) (width 2) (layer B.Cu) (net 12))
 (segment (start 145.161 83.5025) (end 142.494 86.1695) (width 2) (layer B.Cu) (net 12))
 (segment (start 142.4305 86.106) (end 137.7185 86.106) (width 2) (layer B.Cu) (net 12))
 (segment (start 142.494 86.1695) (end 142.4305 86.106) (width 2) (layer B.Cu) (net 12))
 (segment (start 135.763 77.6605) (end 140.081 77.6605) (width 2) (layer B.Cu) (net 13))
 (segment (start 122.9995 90.424) (end 124.587 88.8365) (width 2) (layer B.Cu) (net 13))
 (segment (start 122.9995 93.345) (end 122.9995 90.424) (width 2) (layer B.Cu) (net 13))
 (segment (start 122.8725 90.551) (end 124.587 88.8365) (width 2) (layer B.Cu) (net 13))
 (segment (start 124.587 88.8365) (end 135.763 77.6605) (width 2) (layer B.Cu) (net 13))
 (segment (start 132.140147 89.384353) (end 132.865647 89.384353) (width 0.75) (layer F.Cu) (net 14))
 (segment (start 131.3688 90.1557) (end 132.140147 89.384353) (width 0.75) (layer F.Cu) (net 14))
 (segment (start 132.865647 89.384353) (end 132.889294 89.408) (width 0.75) (layer F.Cu) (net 14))
 (segment (start 132.889294 89.408) (end 148.0185 89.408) (width 0.75) (layer F.Cu) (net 14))
 (segment (start 154.178 83.2485) (end 154.178 77.6605) (width 0.75) (layer B.Cu) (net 14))
 (segment (start 148.0185 89.408) (end 154.178 83.2485) (width 0.75) (layer B.Cu) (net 14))
 (segment (start 148.0185 89.408) (end 148.0185 89.408) (width 0.75) (layer F.Cu) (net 14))
 (via (at 148.0185 89.408) (size 1.4) (drill 0.4) (layers F.Cu B.Cu) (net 14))
 (segment (start 201.422 79.8195) (end 201.422 94.9325) (width 2) (layer B.Cu) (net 15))
 (segment (start 187.96 78.232) (end 199.8345 78.232) (width 2) (layer B.Cu) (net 15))
 (segment (start 199.8345 78.232) (end 201.422 79.8195) (width 2) (layer B.Cu) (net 15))
 (segment (start 177.546 81.153) (end 187.47156 81.153) (width 1) (layer F.Cu) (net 15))
 (segment (start 187.47156 81.153) (end 187.47156 81.153) (width 1) (layer B.Cu) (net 15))
 (via (at 187.47156 81.153) (size 1.4) (drill 0.4) (layers F.Cu B.Cu) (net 15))
 (segment (start 187.96 80.66456) (end 187.70307 80.92149) (width 2) (layer B.Cu) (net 15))
 (segment (start 187.96 77.9145) (end 187.96 80.66456) (width 2) (layer B.Cu) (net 15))
 (segment (start 177.546 81.153) (end 177.546 79.756) (width 1) (layer F.Cu) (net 15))
 (segment (start 177.546 79.756) (end 177.546 79.756) (width 1) (layer B.Cu) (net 15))
 (via (at 177.546 79.756) (size 1.4) (drill 0.4) (layers F.Cu B.Cu) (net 15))
 (segment (start 176.149 79.756) (end 174.117 77.724) (width 1) (layer B.Cu) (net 15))
 (segment (start 177.546 79.756) (end 176.149 79.756) (width 1) (layer B.Cu) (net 15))
 (segment (start 171.1735 101.727) (end 176.7615 107.315) (width 0.8) (layer F.Cu) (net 16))
 (segment (start 170.361 101.727) (end 171.1735 101.727) (width 0.8) (layer F.Cu) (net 16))
 (segment (start 176.7615 107.315) (end 196.215 107.569) (width 0.8) (layer F.Cu) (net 16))
 (segment (start 195.961 107.315) (end 196.215 107.569) (width 0.8) (layer B.Cu) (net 16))
 (segment (start 176.7615 107.315) (end 176.7615 107.315) (width 0.8) (layer F.Cu) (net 16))
 (segment (start 196.215 107.569) (end 195.961 107.315) (width 0.8) (layer B.Cu) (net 16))
 (via (at 196.215 107.569) (size 2) (drill 0.4) (layers F.Cu B.Cu) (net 16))
 (segment (start 196.215 107.569) (end 196.215 110.236) (width 2) (layer B.Cu) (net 16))
 (segment (start 179.197 110.236) (end 177.927 111.506) (width 2) (layer B.Cu) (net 17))
 (segment (start 191.135 110.236) (end 179.197 110.236) (width 2) (layer B.Cu) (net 17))
 (segment (start 171.069 104.648) (end 170.361 104.648) (width 0.8) (layer F.Cu) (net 17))
 (segment (start 177.927 111.506) (end 173.863 107.442) (width 0.8) (layer B.Cu) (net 17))
 (segment (start 173.863 107.442) (end 171.069 104.648) (width 0.8) (layer F.Cu) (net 17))
 (via (at 173.863 107.442) (size 1.4) (drill 0.4) (layers F.Cu B.Cu) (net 17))
 (segment (start 134.62 99.06) (end 137.795 99.06) (width 0.75) (layer F.Cu) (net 3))
 (segment (start 134.42 99.06) (end 131.445 96.085) (width 0.75) (layer F.Cu) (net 3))
 (segment (start 134.62 99.06) (end 134.42 99.06) (width 0.75) (layer F.Cu) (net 3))
 (segment (start 138.77 99.06) (end 144.018 99.06) (width 0.75) (layer F.Cu) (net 3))
 (segment (start 137.795 99.06) (end 138.77 99.06) (width 0.75) (layer F.Cu) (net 3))
 (segment (start 131.445 93.2069) (end 131.3688 93.1307) (width 0.8) (layer F.Cu) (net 3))
 (segment (start 131.445 96.085) (end 131.445 93.2069) (width 0.8) (layer F.Cu) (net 3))
 (segment (start 144.018 99.06) (end 149.86 99.06) (width 0.75) (layer B.Cu) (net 3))
 (via (at 144.018 99.06) (size 1.4) (drill 0.4) (layers F.Cu B.Cu) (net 3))
 (segment (start 167.259 101.6) (end 167.386 101.727) (width 0.75) (layer F.Cu) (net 4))
 (segment (start 157.48 101.6) (end 160.02 101.6) (width 0.75) (layer B.Cu) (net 4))
 (segment (start 160.02 101.6) (end 167.259 101.6) (width 0.75) (layer F.Cu) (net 4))
 (via (at 160.02 101.6) (size 1.4) (drill 0.4) (layers F.Cu B.Cu) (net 4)))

